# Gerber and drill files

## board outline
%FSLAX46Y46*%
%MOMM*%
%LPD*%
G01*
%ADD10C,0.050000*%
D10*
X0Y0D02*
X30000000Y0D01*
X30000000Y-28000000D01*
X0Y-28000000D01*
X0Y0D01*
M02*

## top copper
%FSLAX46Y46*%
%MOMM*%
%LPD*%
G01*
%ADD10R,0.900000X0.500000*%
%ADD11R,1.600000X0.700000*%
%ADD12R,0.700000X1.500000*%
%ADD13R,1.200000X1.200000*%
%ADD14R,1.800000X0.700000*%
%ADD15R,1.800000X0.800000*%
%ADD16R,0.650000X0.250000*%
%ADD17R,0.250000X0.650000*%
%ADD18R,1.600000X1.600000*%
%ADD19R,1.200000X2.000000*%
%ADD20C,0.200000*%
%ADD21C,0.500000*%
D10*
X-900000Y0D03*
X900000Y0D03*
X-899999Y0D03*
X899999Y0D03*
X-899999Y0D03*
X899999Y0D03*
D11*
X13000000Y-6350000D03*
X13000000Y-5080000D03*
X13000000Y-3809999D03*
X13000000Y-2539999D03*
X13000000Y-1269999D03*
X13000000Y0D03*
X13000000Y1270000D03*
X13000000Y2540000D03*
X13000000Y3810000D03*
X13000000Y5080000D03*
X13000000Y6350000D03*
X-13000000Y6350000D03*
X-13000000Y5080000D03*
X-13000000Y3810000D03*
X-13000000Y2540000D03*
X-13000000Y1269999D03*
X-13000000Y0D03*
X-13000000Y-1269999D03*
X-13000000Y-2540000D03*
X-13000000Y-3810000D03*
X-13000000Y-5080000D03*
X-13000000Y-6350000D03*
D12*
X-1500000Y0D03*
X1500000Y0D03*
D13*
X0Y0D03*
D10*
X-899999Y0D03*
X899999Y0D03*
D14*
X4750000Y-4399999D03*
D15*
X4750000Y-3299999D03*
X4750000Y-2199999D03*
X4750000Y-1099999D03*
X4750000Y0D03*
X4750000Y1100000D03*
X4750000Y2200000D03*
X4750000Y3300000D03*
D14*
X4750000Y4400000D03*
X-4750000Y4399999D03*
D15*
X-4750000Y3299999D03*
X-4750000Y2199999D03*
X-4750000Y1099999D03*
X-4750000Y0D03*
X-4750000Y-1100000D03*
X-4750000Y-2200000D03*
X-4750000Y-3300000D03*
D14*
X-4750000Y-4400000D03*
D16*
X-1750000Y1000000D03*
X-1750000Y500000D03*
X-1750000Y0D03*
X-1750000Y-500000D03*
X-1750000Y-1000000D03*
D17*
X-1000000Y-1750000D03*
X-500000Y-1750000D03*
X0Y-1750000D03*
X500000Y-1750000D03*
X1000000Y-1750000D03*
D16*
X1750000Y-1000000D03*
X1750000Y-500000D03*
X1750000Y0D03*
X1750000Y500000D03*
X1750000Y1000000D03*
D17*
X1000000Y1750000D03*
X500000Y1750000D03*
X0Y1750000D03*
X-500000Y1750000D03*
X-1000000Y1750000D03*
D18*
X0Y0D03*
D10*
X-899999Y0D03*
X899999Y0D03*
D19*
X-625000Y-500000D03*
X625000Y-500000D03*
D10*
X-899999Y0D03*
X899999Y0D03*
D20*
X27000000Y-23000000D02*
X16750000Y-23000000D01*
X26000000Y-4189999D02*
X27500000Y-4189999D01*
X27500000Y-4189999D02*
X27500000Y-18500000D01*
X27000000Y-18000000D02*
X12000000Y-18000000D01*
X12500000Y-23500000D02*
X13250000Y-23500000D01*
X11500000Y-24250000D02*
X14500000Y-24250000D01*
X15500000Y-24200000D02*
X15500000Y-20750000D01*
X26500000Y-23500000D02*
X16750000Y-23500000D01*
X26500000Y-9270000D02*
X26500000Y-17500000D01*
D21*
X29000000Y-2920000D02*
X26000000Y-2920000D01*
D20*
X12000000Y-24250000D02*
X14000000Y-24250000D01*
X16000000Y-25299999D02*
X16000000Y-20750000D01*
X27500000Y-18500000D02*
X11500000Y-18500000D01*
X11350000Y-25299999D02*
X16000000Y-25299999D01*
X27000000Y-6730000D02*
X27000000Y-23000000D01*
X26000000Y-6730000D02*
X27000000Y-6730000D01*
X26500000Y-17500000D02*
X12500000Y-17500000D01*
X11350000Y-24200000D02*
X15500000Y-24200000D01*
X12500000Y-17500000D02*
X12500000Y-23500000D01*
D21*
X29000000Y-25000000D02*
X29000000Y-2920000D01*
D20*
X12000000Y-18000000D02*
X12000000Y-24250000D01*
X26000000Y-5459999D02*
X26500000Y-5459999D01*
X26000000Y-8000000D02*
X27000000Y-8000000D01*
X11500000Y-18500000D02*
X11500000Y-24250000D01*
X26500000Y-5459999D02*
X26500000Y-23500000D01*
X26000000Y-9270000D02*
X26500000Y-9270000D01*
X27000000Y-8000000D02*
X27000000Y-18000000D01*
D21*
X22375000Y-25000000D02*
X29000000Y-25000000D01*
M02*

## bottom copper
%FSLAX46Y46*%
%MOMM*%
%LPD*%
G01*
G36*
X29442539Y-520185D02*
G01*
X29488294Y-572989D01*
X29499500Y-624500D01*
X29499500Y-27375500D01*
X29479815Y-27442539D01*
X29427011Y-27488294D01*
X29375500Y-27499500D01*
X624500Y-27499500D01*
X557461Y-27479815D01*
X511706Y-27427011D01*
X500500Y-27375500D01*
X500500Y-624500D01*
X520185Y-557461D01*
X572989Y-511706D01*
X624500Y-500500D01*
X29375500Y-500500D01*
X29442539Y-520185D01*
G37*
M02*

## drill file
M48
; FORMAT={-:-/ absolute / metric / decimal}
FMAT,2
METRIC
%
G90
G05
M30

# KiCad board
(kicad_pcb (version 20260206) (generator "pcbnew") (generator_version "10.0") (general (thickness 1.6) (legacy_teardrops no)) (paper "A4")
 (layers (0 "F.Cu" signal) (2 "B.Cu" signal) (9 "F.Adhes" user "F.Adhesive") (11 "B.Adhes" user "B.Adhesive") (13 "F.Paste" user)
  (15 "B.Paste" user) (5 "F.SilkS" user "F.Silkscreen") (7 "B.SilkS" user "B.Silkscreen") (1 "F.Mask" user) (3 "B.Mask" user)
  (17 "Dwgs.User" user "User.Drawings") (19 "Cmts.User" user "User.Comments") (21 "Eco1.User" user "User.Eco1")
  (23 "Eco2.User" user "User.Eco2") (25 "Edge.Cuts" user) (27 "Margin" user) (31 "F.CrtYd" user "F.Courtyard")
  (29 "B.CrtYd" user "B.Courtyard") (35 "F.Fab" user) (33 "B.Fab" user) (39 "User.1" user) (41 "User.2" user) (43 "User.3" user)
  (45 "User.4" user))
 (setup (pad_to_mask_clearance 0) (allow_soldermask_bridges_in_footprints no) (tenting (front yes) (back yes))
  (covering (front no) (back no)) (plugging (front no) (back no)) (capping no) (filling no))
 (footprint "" (layer "F.Cu") (at 11.5 22)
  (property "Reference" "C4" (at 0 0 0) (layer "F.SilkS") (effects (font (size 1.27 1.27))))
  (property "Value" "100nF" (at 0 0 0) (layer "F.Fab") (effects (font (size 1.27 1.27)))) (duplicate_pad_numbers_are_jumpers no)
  (pad "1" smd rect (at -12.4 -22) (size 0.9 0.5) (layers "F.Cu" "F.Mask" "F.Paste") (thermal_bridge_angle 45))
  (pad "2" smd rect (at -10.6 -22) (size 0.9 0.5) (layers "F.Cu" "F.Mask" "F.Paste") (thermal_bridge_angle 45)))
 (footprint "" (layer "F.Cu") (at 27.5 5.5)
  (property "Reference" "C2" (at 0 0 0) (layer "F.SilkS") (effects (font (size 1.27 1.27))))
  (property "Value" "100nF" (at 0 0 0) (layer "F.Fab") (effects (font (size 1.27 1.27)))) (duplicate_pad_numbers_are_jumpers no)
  (pad "1" smd rect (at -28.399999 -5.5) (size 0.9 0.5) (layers "F.Cu" "F.Mask" "F.Paste") (thermal_bridge_angle 45))
  (pad "2" smd rect (at -26.600001 -5.5) (size 0.9 0.5) (layers "F.Cu" "F.Mask" "F.Paste") (thermal_bridge_angle 45)))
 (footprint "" (layer "F.Cu") (at 27.5 2.5)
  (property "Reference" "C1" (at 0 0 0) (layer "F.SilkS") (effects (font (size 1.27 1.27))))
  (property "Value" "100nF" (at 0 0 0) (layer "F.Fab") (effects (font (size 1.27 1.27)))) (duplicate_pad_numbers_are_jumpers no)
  (pad "1" smd rect (at -28.399999 -2.5) (size 0.9 0.5) (layers "F.Cu" "F.Mask" "F.Paste") (thermal_bridge_angle 45))
  (pad "2" smd rect (at -26.600001 -2.5) (size 0.9 0.5) (layers "F.Cu" "F.Mask" "F.Paste") (thermal_bridge_angle 45)))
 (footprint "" (layer "F.Cu") (at 13 8)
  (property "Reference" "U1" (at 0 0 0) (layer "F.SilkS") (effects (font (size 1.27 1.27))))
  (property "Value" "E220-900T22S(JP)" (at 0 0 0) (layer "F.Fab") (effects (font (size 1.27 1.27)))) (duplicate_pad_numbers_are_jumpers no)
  (pad "1" smd rect (at 0 -1.65) (size 1.6 0.7) (layers "F.Cu" "F.Mask" "F.Paste") (thermal_bridge_angle 45))
  (pad "2" smd rect (at 0 -2.92) (size 1.6 0.7) (layers "F.Cu" "F.Mask" "F.Paste") (thermal_bridge_angle 45))
  (pad "3" smd rect (at 0 -4.190001) (size 1.6 0.7) (layers "F.Cu" "F.Mask" "F.Paste") (thermal_bridge_angle 45))
  (pad "4" smd rect (at 0 -5.460001) (size 1.6 0.7) (layers "F.Cu" "F.Mask" "F.Paste") (thermal_bridge_angle 45))
  (pad "5" smd rect (at 0 -6.730001) (size 1.6 0.7) (layers "F.Cu" "F.Mask" "F.Paste") (thermal_bridge_angle 45))
  (pad "6" smd rect (at 0 -8) (size 1.6 0.7) (layers "F.Cu" "F.Mask" "F.Paste") (thermal_bridge_angle 45))
  (pad "7" smd rect (at 0 -9.27) (size 1.6 0.7) (layers "F.Cu" "F.Mask" "F.Paste") (thermal_bridge_angle 45))
  (pad "8" smd rect (at 0 -10.54) (size 1.6 0.7) (layers "F.Cu" "F.Mask" "F.Paste") (thermal_bridge_angle 45))
  (pad "9" smd rect (at 0 -11.81) (size 1.6 0.7) (layers "F.Cu" "F.Mask" "F.Paste") (thermal_bridge_angle 45))
  (pad "10" smd rect (at 0 -13.08) (size 1.6 0.7) (layers "F.Cu" "F.Mask" "F.Paste") (thermal_bridge_angle 45))
  (pad "11" smd rect (at 0 -14.35) (size 1.6 0.7) (layers "F.Cu" "F.Mask" "F.Paste") (thermal_bridge_angle 45))
  (pad "12" smd rect (at -26 -14.35) (size 1.6 0.7) (layers "F.Cu" "F.Mask" "F.Paste") (thermal_bridge_angle 45))
  (pad "13" smd rect (at -26 -13.08) (size 1.6 0.7) (layers "F.Cu" "F.Mask" "F.Paste") (thermal_bridge_angle 45))
  (pad "14" smd rect (at -26 -11.81) (size 1.6 0.7) (layers "F.Cu" "F.Mask" "F.Paste") (thermal_bridge_angle 45))
  (pad "15" smd rect (at -26 -10.54) (size 1.6 0.7) (layers "F.Cu" "F.Mask" "F.Paste") (thermal_bridge_angle 45))
  (pad "16" smd rect (at -26 -9.269999) (size 1.6 0.7) (layers "F.Cu" "F.Mask" "F.Paste") (thermal_bridge_angle 45))
  (pad "17" smd rect (at -26 -8) (size 1.6 0.7) (layers "F.Cu" "F.Mask" "F.Paste") (thermal_bridge_angle 45))
  (pad "18" smd rect (at -26 -6.730001) (size 1.6 0.7) (layers "F.Cu" "F.Mask" "F.Paste") (thermal_bridge_angle 45))
  (pad "19" smd rect (at -26 -5.46) (size 1.6 0.7) (layers "F.Cu" "F.Mask" "F.Paste") (thermal_bridge_angle 45))
  (pad "20" smd rect (at -26 -4.19) (size 1.6 0.7) (layers "F.Cu" "F.Mask" "F.Paste") (thermal_bridge_angle 45))
  (pad "21" smd rect (at -26 -2.92) (size 1.6 0.7) (layers "F.Cu" "F.Mask" "F.Paste") (thermal_bridge_angle 45))
  (pad "22" smd rect (at -26 -1.65) (size 1.6 0.7) (layers "F.Cu" "F.Mask" "F.Paste") (thermal_bridge_angle 45)))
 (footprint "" (layer "F.Cu") (at 25 19)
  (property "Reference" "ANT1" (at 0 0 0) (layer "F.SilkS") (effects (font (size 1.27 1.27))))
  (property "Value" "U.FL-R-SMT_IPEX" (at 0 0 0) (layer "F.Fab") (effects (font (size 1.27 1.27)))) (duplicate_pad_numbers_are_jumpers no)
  (pad "G1" smd rect (at -26.5 -19) (size 0.7 1.5) (layers "F.Cu" "F.Mask" "F.Paste") (thermal_bridge_angle 45))
  (pad "G2" smd rect (at -23.5 -19) (size 0.7 1.5) (layers "F.Cu" "F.Mask" "F.Paste") (thermal_bridge_angle 45))
  (pad "S" smd rect (at -25 -19) (size 1.2 1.2) (layers "F.Cu" "F.Mask" "F.Paste") (thermal_bridge_angle 45)))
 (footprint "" (layer "F.Cu") (at 19.5 24.5)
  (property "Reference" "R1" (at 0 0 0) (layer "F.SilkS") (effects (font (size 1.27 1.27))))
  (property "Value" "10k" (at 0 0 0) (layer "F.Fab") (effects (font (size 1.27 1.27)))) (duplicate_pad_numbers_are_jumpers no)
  (pad "1" smd rect (at -20.399999 -24.5) (size 0.9 0.5) (layers "F.Cu" "F.Mask" "F.Paste") (thermal_bridge_angle 45))
  (pad "2" smd rect (at -18.600001 -24.5) (size 0.9 0.5) (layers "F.Cu" "F.Mask" "F.Paste") (thermal_bridge_angle 45)))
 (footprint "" (layer "F.Cu") (at 6.6 22)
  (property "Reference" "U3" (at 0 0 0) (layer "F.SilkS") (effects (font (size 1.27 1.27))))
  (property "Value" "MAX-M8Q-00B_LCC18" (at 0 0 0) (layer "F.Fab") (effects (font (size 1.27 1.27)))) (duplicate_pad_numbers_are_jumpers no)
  (pad "1" smd rect (at -1.85 -17.600001) (size 1.8 0.7) (layers "F.Cu" "F.Mask" "F.Paste") (thermal_bridge_angle 45))
  (pad "2" smd rect (at -1.85 -18.700001) (size 1.8 0.8) (layers "F.Cu" "F.Mask" "F.Paste") (thermal_bridge_angle 45))
  (pad "3" smd rect (at -1.85 -19.800001) (size 1.8 0.8) (layers "F.Cu" "F.Mask" "F.Paste") (thermal_bridge_angle 45))
  (pad "4" smd rect (at -1.85 -20.900001) (size 1.8 0.8) (layers "F.Cu" "F.Mask" "F.Paste") (thermal_bridge_angle 45))
  (pad "5" smd rect (at -1.85 -22) (size 1.8 0.8) (layers "F.Cu" "F.Mask" "F.Paste") (thermal_bridge_angle 45))
  (pad "6" smd rect (at -1.85 -23.1) (size 1.8 0.8) (layers "F.Cu" "F.Mask" "F.Paste") (thermal_bridge_angle 45))
  (pad "7" smd rect (at -1.85 -24.2) (size 1.8 0.8) (layers "F.Cu" "F.Mask" "F.Paste") (thermal_bridge_angle 45))
  (pad "8" smd rect (at -1.85 -25.3) (size 1.8 0.8) (layers "F.Cu" "F.Mask" "F.Paste") (thermal_bridge_angle 45))
  (pad "9" smd rect (at -1.85 -26.4) (size 1.8 0.7) (layers "F.Cu" "F.Mask" "F.Paste") (thermal_bridge_angle 45))
  (pad "10" smd rect (at -11.35 -26.399999) (size 1.8 0.7) (layers "F.Cu" "F.Mask" "F.Paste") (thermal_bridge_angle 45))
  (pad "11" smd rect (at -11.35 -25.299999) (size 1.8 0.8) (layers "F.Cu" "F.Mask" "F.Paste") (thermal_bridge_angle 45))
  (pad "12" smd rect (at -11.35 -24.199999) (size 1.8 0.8) (layers "F.Cu" "F.Mask" "F.Paste") (thermal_bridge_angle 45))
  (pad "13" smd rect (at -11.35 -23.099999) (size 1.8 0.8) (layers "F.Cu" "F.Mask" "F.Paste") (thermal_bridge_angle 45))
  (pad "14" smd rect (at -11.35 -22) (size 1.8 0.8) (layers "F.Cu" "F.Mask" "F.Paste") (thermal_bridge_angle 45))
  (pad "15" smd rect (at -11.35 -20.9) (size 1.8 0.8) (layers "F.Cu" "F.Mask" "F.Paste") (thermal_bridge_angle 45))
  (pad "16" smd rect (at -11.35 -19.8) (size 1.8 0.8) (layers "F.Cu" "F.Mask" "F.Paste") (thermal_bridge_angle 45))
  (pad "17" smd rect (at -11.35 -18.7) (size 1.8 0.8) (layers "F.Cu" "F.Mask" "F.Paste") (thermal_bridge_angle 45))
  (pad "18" smd rect (at -11.35 -17.6) (size 1.8 0.7) (layers "F.Cu" "F.Mask" "F.Paste") (thermal_bridge_angle 45)))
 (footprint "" (layer "F.Cu") (at 15 22.5)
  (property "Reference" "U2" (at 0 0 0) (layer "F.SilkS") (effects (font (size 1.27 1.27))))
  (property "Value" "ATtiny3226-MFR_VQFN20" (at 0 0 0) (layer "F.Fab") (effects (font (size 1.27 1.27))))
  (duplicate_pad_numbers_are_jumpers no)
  (pad "1" smd rect (at -16.75 -23.5) (size 0.65 0.25) (layers "F.Cu" "F.Mask" "F.Paste") (thermal_bridge_angle 45))
  (pad "2" smd rect (at -16.75 -23) (size 0.65 0.25) (layers "F.Cu" "F.Mask" "F.Paste") (thermal_bridge_angle 45))
  (pad "3" smd rect (at -16.75 -22.5) (size 0.65 0.25) (layers "F.Cu" "F.Mask" "F.Paste") (thermal_bridge_angle 45))
  (pad "4" smd rect (at -16.75 -22) (size 0.65 0.25) (layers "F.Cu" "F.Mask" "F.Paste") (thermal_bridge_angle 45))
  (pad "5" smd rect (at -16.75 -21.5) (size 0.65 0.25) (layers "F.Cu" "F.Mask" "F.Paste") (thermal_bridge_angle 45))
  (pad "6" smd rect (at -16 -20.75) (size 0.25 0.65) (layers "F.Cu" "F.Mask" "F.Paste") (thermal_bridge_angle 45))
  (pad "7" smd rect (at -15.5 -20.75) (size 0.25 0.65) (layers "F.Cu" "F.Mask" "F.Paste") (thermal_bridge_angle 45))
  (pad "8" smd rect (at -15 -20.75) (size 0.25 0.65) (layers "F.Cu" "F.Mask" "F.Paste") (thermal_bridge_angle 45))
  (pad "9" smd rect (at -14.5 -20.75) (size 0.25 0.65) (layers "F.Cu" "F.Mask" "F.Paste") (thermal_bridge_angle 45))
  (pad "10" smd rect (at -14 -20.75) (size 0.25 0.65) (layers "F.Cu" "F.Mask" "F.Paste") (thermal_bridge_angle 45))
  (pad "11" smd rect (at -13.25 -21.5) (size 0.65 0.25) (layers "F.Cu" "F.Mask" "F.Paste") (thermal_bridge_angle 45))
  (pad "12" smd rect (at -13.25 -22) (size 0.65 0.25) (layers "F.Cu" "F.Mask" "F.Paste") (thermal_bridge_angle 45))
  (pad "13" smd rect (at -13.25 -22.5) (size 0.65 0.25) (layers "F.Cu" "F.Mask" "F.Paste") (thermal_bridge_angle 45))
  (pad "14" smd rect (at -13.25 -23) (size 0.65 0.25) (layers "F.Cu" "F.Mask" "F.Paste") (thermal_bridge_angle 45))
  (pad "15" smd rect (at -13.25 -23.5) (size 0.65 0.25) (layers "F.Cu" "F.Mask" "F.Paste") (thermal_bridge_angle 45))
  (pad "16" smd rect (at -14 -24.25) (size 0.25 0.65) (layers "F.Cu" "F.Mask" "F.Paste") (thermal_bridge_angle 45))
  (pad "17" smd rect (at -14.5 -24.25) (size 0.25 0.65) (layers "F.Cu" "F.Mask" "F.Paste") (thermal_bridge_angle 45))
  (pad "18" smd rect (at -15 -24.25) (size 0.25 0.65) (layers "F.Cu" "F.Mask" "F.Paste") (thermal_bridge_angle 45))
  (pad "19" smd rect (at -15.5 -24.25) (size 0.25 0.65) (layers "F.Cu" "F.Mask" "F.Paste") (thermal_bridge_angle 45))
  (pad "20" smd rect (at -16 -24.25) (size 0.25 0.65) (layers "F.Cu" "F.Mask" "F.Paste") (thermal_bridge_angle 45))
  (pad "EP" smd rect (at -15 -22.5) (size 1.6 1.6) (layers "F.Cu" "F.Mask" "F.Paste") (thermal_bridge_angle 45)))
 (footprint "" (layer "F.Cu") (at 27.5 8.5)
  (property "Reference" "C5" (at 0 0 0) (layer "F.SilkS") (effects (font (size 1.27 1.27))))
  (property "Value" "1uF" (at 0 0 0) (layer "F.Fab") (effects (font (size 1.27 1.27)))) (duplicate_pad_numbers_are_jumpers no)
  (pad "1" smd rect (at -28.399999 -8.5) (size 0.9 0.5) (layers "F.Cu" "F.Mask" "F.Paste") (thermal_bridge_angle 45))
  (pad "2" smd rect (at -26.600001 -8.5) (size 0.9 0.5) (layers "F.Cu" "F.Mask" "F.Paste") (thermal_bridge_angle 45)))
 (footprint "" (layer "F.Cu") (at 23 24.5)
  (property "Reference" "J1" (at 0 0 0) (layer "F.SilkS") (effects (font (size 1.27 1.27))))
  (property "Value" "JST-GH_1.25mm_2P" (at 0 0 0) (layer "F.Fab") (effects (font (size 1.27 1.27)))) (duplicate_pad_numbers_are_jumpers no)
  (pad "1" smd rect (at -23.625 -24) (size 1.2 2) (layers "F.Cu" "F.Mask" "F.Paste") (thermal_bridge_angle 45))
  (pad "2" smd rect (at -22.375 -24) (size 1.2 2) (layers "F.Cu" "F.Mask" "F.Paste") (thermal_bridge_angle 45)))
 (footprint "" (layer "F.Cu") (at 19.5 20.5)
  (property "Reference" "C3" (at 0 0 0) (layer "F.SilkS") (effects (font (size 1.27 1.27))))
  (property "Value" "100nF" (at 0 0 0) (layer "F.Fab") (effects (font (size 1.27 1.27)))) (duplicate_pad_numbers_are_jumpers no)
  (pad "1" smd rect (at -20.399999 -20.5) (size 0.9 0.5) (layers "F.Cu" "F.Mask" "F.Paste") (thermal_bridge_angle 45))
  (pad "2" smd rect (at -18.600001 -20.5) (size 0.9 0.5) (layers "F.Cu" "F.Mask" "F.Paste") (thermal_bridge_angle 45)))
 (gr_rect (start 0 0) (end 30 28) (stroke (width 0.05) (type default)) (fill no) (layer "Edge.Cuts"))
 (segment (start 27 23) (end 16.75 23) (width 0.2) (layer "F.Cu") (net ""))
 (segment (start 26 4.189999) (end 27.5 4.189999) (width 0.2) (layer "F.Cu") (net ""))
 (segment (start 27.5 4.189999) (end 27.5 18.5) (width 0.2) (layer "F.Cu") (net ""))
 (segment (start 27 18) (end 12 18) (width 0.2) (layer "F.Cu") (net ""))
 (segment (start 12.5 23.5) (end 13.25 23.5) (width 0.2) (layer "F.Cu") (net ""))
 (segment (start 11.5 24.25) (end 14.5 24.25) (width 0.2) (layer "F.Cu") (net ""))
 (segment (start 15.5 24.2) (end 15.5 20.75) (width 0.2) (layer "F.Cu") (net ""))
 (segment (start 26.5 23.5) (end 16.75 23.5) (width 0.2) (layer "F.Cu") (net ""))
 (segment (start 26.5 9.27) (end 26.5 17.5) (width 0.2) (layer "F.Cu") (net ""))
 (segment (start 29 2.92) (end 26 2.92) (width 0.5) (layer "F.Cu") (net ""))
 (segment (start 12 24.25) (end 14 24.25) (width 0.2) (layer "F.Cu") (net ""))
 (segment (start 16 25.299999) (end 16 20.75) (width 0.2) (layer "F.Cu") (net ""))
 (segment (start 27.5 18.5) (end 11.5 18.5) (width 0.2) (layer "F.Cu") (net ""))
 (segment (start 11.35 25.299999) (end 16 25.299999) (width 0.2) (layer "F.Cu") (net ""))
 (segment (start 27 6.73) (end 27 23) (width 0.2) (layer "F.Cu") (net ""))
 (segment (start 26 6.73) (end 27 6.73) (width 0.2) (layer "F.Cu") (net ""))
 (segment (start 26.5 17.5) (end 12.5 17.5) (width 0.2) (layer "F.Cu") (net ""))
 (segment (start 11.35 24.2) (end 15.5 24.2) (width 0.2) (layer "F.Cu") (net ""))
 (segment (start 12.5 17.5) (end 12.5 23.5) (width 0.2) (layer "F.Cu") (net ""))
 (segment (start 29 25) (end 29 2.92) (width 0.5) (layer "F.Cu") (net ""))
 (segment (start 12 18) (end 12 24.25) (width 0.2) (layer "F.Cu") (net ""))
 (segment (start 26 5.459999) (end 26.5 5.459999) (width 0.2) (layer "F.Cu") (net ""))
 (segment (start 26 8) (end 27 8) (width 0.2) (layer "F.Cu") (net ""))
 (segment (start 11.5 18.5) (end 11.5 24.25) (width 0.2) (layer "F.Cu") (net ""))
 (segment (start 26.5 5.459999) (end 26.5 23.5) (width 0.2) (layer "F.Cu") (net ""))
 (segment (start 26 9.27) (end 26.5 9.27) (width 0.2) (layer "F.Cu") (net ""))
 (segment (start 27 8) (end 27 18) (width 0.2) (layer "F.Cu") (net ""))
 (segment (start 22.375 25) (end 29 25) (width 0.5) (layer "F.Cu") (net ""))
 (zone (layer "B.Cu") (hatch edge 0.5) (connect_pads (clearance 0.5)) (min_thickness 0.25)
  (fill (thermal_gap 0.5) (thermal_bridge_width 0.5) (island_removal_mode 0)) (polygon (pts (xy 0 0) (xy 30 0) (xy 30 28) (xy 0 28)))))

